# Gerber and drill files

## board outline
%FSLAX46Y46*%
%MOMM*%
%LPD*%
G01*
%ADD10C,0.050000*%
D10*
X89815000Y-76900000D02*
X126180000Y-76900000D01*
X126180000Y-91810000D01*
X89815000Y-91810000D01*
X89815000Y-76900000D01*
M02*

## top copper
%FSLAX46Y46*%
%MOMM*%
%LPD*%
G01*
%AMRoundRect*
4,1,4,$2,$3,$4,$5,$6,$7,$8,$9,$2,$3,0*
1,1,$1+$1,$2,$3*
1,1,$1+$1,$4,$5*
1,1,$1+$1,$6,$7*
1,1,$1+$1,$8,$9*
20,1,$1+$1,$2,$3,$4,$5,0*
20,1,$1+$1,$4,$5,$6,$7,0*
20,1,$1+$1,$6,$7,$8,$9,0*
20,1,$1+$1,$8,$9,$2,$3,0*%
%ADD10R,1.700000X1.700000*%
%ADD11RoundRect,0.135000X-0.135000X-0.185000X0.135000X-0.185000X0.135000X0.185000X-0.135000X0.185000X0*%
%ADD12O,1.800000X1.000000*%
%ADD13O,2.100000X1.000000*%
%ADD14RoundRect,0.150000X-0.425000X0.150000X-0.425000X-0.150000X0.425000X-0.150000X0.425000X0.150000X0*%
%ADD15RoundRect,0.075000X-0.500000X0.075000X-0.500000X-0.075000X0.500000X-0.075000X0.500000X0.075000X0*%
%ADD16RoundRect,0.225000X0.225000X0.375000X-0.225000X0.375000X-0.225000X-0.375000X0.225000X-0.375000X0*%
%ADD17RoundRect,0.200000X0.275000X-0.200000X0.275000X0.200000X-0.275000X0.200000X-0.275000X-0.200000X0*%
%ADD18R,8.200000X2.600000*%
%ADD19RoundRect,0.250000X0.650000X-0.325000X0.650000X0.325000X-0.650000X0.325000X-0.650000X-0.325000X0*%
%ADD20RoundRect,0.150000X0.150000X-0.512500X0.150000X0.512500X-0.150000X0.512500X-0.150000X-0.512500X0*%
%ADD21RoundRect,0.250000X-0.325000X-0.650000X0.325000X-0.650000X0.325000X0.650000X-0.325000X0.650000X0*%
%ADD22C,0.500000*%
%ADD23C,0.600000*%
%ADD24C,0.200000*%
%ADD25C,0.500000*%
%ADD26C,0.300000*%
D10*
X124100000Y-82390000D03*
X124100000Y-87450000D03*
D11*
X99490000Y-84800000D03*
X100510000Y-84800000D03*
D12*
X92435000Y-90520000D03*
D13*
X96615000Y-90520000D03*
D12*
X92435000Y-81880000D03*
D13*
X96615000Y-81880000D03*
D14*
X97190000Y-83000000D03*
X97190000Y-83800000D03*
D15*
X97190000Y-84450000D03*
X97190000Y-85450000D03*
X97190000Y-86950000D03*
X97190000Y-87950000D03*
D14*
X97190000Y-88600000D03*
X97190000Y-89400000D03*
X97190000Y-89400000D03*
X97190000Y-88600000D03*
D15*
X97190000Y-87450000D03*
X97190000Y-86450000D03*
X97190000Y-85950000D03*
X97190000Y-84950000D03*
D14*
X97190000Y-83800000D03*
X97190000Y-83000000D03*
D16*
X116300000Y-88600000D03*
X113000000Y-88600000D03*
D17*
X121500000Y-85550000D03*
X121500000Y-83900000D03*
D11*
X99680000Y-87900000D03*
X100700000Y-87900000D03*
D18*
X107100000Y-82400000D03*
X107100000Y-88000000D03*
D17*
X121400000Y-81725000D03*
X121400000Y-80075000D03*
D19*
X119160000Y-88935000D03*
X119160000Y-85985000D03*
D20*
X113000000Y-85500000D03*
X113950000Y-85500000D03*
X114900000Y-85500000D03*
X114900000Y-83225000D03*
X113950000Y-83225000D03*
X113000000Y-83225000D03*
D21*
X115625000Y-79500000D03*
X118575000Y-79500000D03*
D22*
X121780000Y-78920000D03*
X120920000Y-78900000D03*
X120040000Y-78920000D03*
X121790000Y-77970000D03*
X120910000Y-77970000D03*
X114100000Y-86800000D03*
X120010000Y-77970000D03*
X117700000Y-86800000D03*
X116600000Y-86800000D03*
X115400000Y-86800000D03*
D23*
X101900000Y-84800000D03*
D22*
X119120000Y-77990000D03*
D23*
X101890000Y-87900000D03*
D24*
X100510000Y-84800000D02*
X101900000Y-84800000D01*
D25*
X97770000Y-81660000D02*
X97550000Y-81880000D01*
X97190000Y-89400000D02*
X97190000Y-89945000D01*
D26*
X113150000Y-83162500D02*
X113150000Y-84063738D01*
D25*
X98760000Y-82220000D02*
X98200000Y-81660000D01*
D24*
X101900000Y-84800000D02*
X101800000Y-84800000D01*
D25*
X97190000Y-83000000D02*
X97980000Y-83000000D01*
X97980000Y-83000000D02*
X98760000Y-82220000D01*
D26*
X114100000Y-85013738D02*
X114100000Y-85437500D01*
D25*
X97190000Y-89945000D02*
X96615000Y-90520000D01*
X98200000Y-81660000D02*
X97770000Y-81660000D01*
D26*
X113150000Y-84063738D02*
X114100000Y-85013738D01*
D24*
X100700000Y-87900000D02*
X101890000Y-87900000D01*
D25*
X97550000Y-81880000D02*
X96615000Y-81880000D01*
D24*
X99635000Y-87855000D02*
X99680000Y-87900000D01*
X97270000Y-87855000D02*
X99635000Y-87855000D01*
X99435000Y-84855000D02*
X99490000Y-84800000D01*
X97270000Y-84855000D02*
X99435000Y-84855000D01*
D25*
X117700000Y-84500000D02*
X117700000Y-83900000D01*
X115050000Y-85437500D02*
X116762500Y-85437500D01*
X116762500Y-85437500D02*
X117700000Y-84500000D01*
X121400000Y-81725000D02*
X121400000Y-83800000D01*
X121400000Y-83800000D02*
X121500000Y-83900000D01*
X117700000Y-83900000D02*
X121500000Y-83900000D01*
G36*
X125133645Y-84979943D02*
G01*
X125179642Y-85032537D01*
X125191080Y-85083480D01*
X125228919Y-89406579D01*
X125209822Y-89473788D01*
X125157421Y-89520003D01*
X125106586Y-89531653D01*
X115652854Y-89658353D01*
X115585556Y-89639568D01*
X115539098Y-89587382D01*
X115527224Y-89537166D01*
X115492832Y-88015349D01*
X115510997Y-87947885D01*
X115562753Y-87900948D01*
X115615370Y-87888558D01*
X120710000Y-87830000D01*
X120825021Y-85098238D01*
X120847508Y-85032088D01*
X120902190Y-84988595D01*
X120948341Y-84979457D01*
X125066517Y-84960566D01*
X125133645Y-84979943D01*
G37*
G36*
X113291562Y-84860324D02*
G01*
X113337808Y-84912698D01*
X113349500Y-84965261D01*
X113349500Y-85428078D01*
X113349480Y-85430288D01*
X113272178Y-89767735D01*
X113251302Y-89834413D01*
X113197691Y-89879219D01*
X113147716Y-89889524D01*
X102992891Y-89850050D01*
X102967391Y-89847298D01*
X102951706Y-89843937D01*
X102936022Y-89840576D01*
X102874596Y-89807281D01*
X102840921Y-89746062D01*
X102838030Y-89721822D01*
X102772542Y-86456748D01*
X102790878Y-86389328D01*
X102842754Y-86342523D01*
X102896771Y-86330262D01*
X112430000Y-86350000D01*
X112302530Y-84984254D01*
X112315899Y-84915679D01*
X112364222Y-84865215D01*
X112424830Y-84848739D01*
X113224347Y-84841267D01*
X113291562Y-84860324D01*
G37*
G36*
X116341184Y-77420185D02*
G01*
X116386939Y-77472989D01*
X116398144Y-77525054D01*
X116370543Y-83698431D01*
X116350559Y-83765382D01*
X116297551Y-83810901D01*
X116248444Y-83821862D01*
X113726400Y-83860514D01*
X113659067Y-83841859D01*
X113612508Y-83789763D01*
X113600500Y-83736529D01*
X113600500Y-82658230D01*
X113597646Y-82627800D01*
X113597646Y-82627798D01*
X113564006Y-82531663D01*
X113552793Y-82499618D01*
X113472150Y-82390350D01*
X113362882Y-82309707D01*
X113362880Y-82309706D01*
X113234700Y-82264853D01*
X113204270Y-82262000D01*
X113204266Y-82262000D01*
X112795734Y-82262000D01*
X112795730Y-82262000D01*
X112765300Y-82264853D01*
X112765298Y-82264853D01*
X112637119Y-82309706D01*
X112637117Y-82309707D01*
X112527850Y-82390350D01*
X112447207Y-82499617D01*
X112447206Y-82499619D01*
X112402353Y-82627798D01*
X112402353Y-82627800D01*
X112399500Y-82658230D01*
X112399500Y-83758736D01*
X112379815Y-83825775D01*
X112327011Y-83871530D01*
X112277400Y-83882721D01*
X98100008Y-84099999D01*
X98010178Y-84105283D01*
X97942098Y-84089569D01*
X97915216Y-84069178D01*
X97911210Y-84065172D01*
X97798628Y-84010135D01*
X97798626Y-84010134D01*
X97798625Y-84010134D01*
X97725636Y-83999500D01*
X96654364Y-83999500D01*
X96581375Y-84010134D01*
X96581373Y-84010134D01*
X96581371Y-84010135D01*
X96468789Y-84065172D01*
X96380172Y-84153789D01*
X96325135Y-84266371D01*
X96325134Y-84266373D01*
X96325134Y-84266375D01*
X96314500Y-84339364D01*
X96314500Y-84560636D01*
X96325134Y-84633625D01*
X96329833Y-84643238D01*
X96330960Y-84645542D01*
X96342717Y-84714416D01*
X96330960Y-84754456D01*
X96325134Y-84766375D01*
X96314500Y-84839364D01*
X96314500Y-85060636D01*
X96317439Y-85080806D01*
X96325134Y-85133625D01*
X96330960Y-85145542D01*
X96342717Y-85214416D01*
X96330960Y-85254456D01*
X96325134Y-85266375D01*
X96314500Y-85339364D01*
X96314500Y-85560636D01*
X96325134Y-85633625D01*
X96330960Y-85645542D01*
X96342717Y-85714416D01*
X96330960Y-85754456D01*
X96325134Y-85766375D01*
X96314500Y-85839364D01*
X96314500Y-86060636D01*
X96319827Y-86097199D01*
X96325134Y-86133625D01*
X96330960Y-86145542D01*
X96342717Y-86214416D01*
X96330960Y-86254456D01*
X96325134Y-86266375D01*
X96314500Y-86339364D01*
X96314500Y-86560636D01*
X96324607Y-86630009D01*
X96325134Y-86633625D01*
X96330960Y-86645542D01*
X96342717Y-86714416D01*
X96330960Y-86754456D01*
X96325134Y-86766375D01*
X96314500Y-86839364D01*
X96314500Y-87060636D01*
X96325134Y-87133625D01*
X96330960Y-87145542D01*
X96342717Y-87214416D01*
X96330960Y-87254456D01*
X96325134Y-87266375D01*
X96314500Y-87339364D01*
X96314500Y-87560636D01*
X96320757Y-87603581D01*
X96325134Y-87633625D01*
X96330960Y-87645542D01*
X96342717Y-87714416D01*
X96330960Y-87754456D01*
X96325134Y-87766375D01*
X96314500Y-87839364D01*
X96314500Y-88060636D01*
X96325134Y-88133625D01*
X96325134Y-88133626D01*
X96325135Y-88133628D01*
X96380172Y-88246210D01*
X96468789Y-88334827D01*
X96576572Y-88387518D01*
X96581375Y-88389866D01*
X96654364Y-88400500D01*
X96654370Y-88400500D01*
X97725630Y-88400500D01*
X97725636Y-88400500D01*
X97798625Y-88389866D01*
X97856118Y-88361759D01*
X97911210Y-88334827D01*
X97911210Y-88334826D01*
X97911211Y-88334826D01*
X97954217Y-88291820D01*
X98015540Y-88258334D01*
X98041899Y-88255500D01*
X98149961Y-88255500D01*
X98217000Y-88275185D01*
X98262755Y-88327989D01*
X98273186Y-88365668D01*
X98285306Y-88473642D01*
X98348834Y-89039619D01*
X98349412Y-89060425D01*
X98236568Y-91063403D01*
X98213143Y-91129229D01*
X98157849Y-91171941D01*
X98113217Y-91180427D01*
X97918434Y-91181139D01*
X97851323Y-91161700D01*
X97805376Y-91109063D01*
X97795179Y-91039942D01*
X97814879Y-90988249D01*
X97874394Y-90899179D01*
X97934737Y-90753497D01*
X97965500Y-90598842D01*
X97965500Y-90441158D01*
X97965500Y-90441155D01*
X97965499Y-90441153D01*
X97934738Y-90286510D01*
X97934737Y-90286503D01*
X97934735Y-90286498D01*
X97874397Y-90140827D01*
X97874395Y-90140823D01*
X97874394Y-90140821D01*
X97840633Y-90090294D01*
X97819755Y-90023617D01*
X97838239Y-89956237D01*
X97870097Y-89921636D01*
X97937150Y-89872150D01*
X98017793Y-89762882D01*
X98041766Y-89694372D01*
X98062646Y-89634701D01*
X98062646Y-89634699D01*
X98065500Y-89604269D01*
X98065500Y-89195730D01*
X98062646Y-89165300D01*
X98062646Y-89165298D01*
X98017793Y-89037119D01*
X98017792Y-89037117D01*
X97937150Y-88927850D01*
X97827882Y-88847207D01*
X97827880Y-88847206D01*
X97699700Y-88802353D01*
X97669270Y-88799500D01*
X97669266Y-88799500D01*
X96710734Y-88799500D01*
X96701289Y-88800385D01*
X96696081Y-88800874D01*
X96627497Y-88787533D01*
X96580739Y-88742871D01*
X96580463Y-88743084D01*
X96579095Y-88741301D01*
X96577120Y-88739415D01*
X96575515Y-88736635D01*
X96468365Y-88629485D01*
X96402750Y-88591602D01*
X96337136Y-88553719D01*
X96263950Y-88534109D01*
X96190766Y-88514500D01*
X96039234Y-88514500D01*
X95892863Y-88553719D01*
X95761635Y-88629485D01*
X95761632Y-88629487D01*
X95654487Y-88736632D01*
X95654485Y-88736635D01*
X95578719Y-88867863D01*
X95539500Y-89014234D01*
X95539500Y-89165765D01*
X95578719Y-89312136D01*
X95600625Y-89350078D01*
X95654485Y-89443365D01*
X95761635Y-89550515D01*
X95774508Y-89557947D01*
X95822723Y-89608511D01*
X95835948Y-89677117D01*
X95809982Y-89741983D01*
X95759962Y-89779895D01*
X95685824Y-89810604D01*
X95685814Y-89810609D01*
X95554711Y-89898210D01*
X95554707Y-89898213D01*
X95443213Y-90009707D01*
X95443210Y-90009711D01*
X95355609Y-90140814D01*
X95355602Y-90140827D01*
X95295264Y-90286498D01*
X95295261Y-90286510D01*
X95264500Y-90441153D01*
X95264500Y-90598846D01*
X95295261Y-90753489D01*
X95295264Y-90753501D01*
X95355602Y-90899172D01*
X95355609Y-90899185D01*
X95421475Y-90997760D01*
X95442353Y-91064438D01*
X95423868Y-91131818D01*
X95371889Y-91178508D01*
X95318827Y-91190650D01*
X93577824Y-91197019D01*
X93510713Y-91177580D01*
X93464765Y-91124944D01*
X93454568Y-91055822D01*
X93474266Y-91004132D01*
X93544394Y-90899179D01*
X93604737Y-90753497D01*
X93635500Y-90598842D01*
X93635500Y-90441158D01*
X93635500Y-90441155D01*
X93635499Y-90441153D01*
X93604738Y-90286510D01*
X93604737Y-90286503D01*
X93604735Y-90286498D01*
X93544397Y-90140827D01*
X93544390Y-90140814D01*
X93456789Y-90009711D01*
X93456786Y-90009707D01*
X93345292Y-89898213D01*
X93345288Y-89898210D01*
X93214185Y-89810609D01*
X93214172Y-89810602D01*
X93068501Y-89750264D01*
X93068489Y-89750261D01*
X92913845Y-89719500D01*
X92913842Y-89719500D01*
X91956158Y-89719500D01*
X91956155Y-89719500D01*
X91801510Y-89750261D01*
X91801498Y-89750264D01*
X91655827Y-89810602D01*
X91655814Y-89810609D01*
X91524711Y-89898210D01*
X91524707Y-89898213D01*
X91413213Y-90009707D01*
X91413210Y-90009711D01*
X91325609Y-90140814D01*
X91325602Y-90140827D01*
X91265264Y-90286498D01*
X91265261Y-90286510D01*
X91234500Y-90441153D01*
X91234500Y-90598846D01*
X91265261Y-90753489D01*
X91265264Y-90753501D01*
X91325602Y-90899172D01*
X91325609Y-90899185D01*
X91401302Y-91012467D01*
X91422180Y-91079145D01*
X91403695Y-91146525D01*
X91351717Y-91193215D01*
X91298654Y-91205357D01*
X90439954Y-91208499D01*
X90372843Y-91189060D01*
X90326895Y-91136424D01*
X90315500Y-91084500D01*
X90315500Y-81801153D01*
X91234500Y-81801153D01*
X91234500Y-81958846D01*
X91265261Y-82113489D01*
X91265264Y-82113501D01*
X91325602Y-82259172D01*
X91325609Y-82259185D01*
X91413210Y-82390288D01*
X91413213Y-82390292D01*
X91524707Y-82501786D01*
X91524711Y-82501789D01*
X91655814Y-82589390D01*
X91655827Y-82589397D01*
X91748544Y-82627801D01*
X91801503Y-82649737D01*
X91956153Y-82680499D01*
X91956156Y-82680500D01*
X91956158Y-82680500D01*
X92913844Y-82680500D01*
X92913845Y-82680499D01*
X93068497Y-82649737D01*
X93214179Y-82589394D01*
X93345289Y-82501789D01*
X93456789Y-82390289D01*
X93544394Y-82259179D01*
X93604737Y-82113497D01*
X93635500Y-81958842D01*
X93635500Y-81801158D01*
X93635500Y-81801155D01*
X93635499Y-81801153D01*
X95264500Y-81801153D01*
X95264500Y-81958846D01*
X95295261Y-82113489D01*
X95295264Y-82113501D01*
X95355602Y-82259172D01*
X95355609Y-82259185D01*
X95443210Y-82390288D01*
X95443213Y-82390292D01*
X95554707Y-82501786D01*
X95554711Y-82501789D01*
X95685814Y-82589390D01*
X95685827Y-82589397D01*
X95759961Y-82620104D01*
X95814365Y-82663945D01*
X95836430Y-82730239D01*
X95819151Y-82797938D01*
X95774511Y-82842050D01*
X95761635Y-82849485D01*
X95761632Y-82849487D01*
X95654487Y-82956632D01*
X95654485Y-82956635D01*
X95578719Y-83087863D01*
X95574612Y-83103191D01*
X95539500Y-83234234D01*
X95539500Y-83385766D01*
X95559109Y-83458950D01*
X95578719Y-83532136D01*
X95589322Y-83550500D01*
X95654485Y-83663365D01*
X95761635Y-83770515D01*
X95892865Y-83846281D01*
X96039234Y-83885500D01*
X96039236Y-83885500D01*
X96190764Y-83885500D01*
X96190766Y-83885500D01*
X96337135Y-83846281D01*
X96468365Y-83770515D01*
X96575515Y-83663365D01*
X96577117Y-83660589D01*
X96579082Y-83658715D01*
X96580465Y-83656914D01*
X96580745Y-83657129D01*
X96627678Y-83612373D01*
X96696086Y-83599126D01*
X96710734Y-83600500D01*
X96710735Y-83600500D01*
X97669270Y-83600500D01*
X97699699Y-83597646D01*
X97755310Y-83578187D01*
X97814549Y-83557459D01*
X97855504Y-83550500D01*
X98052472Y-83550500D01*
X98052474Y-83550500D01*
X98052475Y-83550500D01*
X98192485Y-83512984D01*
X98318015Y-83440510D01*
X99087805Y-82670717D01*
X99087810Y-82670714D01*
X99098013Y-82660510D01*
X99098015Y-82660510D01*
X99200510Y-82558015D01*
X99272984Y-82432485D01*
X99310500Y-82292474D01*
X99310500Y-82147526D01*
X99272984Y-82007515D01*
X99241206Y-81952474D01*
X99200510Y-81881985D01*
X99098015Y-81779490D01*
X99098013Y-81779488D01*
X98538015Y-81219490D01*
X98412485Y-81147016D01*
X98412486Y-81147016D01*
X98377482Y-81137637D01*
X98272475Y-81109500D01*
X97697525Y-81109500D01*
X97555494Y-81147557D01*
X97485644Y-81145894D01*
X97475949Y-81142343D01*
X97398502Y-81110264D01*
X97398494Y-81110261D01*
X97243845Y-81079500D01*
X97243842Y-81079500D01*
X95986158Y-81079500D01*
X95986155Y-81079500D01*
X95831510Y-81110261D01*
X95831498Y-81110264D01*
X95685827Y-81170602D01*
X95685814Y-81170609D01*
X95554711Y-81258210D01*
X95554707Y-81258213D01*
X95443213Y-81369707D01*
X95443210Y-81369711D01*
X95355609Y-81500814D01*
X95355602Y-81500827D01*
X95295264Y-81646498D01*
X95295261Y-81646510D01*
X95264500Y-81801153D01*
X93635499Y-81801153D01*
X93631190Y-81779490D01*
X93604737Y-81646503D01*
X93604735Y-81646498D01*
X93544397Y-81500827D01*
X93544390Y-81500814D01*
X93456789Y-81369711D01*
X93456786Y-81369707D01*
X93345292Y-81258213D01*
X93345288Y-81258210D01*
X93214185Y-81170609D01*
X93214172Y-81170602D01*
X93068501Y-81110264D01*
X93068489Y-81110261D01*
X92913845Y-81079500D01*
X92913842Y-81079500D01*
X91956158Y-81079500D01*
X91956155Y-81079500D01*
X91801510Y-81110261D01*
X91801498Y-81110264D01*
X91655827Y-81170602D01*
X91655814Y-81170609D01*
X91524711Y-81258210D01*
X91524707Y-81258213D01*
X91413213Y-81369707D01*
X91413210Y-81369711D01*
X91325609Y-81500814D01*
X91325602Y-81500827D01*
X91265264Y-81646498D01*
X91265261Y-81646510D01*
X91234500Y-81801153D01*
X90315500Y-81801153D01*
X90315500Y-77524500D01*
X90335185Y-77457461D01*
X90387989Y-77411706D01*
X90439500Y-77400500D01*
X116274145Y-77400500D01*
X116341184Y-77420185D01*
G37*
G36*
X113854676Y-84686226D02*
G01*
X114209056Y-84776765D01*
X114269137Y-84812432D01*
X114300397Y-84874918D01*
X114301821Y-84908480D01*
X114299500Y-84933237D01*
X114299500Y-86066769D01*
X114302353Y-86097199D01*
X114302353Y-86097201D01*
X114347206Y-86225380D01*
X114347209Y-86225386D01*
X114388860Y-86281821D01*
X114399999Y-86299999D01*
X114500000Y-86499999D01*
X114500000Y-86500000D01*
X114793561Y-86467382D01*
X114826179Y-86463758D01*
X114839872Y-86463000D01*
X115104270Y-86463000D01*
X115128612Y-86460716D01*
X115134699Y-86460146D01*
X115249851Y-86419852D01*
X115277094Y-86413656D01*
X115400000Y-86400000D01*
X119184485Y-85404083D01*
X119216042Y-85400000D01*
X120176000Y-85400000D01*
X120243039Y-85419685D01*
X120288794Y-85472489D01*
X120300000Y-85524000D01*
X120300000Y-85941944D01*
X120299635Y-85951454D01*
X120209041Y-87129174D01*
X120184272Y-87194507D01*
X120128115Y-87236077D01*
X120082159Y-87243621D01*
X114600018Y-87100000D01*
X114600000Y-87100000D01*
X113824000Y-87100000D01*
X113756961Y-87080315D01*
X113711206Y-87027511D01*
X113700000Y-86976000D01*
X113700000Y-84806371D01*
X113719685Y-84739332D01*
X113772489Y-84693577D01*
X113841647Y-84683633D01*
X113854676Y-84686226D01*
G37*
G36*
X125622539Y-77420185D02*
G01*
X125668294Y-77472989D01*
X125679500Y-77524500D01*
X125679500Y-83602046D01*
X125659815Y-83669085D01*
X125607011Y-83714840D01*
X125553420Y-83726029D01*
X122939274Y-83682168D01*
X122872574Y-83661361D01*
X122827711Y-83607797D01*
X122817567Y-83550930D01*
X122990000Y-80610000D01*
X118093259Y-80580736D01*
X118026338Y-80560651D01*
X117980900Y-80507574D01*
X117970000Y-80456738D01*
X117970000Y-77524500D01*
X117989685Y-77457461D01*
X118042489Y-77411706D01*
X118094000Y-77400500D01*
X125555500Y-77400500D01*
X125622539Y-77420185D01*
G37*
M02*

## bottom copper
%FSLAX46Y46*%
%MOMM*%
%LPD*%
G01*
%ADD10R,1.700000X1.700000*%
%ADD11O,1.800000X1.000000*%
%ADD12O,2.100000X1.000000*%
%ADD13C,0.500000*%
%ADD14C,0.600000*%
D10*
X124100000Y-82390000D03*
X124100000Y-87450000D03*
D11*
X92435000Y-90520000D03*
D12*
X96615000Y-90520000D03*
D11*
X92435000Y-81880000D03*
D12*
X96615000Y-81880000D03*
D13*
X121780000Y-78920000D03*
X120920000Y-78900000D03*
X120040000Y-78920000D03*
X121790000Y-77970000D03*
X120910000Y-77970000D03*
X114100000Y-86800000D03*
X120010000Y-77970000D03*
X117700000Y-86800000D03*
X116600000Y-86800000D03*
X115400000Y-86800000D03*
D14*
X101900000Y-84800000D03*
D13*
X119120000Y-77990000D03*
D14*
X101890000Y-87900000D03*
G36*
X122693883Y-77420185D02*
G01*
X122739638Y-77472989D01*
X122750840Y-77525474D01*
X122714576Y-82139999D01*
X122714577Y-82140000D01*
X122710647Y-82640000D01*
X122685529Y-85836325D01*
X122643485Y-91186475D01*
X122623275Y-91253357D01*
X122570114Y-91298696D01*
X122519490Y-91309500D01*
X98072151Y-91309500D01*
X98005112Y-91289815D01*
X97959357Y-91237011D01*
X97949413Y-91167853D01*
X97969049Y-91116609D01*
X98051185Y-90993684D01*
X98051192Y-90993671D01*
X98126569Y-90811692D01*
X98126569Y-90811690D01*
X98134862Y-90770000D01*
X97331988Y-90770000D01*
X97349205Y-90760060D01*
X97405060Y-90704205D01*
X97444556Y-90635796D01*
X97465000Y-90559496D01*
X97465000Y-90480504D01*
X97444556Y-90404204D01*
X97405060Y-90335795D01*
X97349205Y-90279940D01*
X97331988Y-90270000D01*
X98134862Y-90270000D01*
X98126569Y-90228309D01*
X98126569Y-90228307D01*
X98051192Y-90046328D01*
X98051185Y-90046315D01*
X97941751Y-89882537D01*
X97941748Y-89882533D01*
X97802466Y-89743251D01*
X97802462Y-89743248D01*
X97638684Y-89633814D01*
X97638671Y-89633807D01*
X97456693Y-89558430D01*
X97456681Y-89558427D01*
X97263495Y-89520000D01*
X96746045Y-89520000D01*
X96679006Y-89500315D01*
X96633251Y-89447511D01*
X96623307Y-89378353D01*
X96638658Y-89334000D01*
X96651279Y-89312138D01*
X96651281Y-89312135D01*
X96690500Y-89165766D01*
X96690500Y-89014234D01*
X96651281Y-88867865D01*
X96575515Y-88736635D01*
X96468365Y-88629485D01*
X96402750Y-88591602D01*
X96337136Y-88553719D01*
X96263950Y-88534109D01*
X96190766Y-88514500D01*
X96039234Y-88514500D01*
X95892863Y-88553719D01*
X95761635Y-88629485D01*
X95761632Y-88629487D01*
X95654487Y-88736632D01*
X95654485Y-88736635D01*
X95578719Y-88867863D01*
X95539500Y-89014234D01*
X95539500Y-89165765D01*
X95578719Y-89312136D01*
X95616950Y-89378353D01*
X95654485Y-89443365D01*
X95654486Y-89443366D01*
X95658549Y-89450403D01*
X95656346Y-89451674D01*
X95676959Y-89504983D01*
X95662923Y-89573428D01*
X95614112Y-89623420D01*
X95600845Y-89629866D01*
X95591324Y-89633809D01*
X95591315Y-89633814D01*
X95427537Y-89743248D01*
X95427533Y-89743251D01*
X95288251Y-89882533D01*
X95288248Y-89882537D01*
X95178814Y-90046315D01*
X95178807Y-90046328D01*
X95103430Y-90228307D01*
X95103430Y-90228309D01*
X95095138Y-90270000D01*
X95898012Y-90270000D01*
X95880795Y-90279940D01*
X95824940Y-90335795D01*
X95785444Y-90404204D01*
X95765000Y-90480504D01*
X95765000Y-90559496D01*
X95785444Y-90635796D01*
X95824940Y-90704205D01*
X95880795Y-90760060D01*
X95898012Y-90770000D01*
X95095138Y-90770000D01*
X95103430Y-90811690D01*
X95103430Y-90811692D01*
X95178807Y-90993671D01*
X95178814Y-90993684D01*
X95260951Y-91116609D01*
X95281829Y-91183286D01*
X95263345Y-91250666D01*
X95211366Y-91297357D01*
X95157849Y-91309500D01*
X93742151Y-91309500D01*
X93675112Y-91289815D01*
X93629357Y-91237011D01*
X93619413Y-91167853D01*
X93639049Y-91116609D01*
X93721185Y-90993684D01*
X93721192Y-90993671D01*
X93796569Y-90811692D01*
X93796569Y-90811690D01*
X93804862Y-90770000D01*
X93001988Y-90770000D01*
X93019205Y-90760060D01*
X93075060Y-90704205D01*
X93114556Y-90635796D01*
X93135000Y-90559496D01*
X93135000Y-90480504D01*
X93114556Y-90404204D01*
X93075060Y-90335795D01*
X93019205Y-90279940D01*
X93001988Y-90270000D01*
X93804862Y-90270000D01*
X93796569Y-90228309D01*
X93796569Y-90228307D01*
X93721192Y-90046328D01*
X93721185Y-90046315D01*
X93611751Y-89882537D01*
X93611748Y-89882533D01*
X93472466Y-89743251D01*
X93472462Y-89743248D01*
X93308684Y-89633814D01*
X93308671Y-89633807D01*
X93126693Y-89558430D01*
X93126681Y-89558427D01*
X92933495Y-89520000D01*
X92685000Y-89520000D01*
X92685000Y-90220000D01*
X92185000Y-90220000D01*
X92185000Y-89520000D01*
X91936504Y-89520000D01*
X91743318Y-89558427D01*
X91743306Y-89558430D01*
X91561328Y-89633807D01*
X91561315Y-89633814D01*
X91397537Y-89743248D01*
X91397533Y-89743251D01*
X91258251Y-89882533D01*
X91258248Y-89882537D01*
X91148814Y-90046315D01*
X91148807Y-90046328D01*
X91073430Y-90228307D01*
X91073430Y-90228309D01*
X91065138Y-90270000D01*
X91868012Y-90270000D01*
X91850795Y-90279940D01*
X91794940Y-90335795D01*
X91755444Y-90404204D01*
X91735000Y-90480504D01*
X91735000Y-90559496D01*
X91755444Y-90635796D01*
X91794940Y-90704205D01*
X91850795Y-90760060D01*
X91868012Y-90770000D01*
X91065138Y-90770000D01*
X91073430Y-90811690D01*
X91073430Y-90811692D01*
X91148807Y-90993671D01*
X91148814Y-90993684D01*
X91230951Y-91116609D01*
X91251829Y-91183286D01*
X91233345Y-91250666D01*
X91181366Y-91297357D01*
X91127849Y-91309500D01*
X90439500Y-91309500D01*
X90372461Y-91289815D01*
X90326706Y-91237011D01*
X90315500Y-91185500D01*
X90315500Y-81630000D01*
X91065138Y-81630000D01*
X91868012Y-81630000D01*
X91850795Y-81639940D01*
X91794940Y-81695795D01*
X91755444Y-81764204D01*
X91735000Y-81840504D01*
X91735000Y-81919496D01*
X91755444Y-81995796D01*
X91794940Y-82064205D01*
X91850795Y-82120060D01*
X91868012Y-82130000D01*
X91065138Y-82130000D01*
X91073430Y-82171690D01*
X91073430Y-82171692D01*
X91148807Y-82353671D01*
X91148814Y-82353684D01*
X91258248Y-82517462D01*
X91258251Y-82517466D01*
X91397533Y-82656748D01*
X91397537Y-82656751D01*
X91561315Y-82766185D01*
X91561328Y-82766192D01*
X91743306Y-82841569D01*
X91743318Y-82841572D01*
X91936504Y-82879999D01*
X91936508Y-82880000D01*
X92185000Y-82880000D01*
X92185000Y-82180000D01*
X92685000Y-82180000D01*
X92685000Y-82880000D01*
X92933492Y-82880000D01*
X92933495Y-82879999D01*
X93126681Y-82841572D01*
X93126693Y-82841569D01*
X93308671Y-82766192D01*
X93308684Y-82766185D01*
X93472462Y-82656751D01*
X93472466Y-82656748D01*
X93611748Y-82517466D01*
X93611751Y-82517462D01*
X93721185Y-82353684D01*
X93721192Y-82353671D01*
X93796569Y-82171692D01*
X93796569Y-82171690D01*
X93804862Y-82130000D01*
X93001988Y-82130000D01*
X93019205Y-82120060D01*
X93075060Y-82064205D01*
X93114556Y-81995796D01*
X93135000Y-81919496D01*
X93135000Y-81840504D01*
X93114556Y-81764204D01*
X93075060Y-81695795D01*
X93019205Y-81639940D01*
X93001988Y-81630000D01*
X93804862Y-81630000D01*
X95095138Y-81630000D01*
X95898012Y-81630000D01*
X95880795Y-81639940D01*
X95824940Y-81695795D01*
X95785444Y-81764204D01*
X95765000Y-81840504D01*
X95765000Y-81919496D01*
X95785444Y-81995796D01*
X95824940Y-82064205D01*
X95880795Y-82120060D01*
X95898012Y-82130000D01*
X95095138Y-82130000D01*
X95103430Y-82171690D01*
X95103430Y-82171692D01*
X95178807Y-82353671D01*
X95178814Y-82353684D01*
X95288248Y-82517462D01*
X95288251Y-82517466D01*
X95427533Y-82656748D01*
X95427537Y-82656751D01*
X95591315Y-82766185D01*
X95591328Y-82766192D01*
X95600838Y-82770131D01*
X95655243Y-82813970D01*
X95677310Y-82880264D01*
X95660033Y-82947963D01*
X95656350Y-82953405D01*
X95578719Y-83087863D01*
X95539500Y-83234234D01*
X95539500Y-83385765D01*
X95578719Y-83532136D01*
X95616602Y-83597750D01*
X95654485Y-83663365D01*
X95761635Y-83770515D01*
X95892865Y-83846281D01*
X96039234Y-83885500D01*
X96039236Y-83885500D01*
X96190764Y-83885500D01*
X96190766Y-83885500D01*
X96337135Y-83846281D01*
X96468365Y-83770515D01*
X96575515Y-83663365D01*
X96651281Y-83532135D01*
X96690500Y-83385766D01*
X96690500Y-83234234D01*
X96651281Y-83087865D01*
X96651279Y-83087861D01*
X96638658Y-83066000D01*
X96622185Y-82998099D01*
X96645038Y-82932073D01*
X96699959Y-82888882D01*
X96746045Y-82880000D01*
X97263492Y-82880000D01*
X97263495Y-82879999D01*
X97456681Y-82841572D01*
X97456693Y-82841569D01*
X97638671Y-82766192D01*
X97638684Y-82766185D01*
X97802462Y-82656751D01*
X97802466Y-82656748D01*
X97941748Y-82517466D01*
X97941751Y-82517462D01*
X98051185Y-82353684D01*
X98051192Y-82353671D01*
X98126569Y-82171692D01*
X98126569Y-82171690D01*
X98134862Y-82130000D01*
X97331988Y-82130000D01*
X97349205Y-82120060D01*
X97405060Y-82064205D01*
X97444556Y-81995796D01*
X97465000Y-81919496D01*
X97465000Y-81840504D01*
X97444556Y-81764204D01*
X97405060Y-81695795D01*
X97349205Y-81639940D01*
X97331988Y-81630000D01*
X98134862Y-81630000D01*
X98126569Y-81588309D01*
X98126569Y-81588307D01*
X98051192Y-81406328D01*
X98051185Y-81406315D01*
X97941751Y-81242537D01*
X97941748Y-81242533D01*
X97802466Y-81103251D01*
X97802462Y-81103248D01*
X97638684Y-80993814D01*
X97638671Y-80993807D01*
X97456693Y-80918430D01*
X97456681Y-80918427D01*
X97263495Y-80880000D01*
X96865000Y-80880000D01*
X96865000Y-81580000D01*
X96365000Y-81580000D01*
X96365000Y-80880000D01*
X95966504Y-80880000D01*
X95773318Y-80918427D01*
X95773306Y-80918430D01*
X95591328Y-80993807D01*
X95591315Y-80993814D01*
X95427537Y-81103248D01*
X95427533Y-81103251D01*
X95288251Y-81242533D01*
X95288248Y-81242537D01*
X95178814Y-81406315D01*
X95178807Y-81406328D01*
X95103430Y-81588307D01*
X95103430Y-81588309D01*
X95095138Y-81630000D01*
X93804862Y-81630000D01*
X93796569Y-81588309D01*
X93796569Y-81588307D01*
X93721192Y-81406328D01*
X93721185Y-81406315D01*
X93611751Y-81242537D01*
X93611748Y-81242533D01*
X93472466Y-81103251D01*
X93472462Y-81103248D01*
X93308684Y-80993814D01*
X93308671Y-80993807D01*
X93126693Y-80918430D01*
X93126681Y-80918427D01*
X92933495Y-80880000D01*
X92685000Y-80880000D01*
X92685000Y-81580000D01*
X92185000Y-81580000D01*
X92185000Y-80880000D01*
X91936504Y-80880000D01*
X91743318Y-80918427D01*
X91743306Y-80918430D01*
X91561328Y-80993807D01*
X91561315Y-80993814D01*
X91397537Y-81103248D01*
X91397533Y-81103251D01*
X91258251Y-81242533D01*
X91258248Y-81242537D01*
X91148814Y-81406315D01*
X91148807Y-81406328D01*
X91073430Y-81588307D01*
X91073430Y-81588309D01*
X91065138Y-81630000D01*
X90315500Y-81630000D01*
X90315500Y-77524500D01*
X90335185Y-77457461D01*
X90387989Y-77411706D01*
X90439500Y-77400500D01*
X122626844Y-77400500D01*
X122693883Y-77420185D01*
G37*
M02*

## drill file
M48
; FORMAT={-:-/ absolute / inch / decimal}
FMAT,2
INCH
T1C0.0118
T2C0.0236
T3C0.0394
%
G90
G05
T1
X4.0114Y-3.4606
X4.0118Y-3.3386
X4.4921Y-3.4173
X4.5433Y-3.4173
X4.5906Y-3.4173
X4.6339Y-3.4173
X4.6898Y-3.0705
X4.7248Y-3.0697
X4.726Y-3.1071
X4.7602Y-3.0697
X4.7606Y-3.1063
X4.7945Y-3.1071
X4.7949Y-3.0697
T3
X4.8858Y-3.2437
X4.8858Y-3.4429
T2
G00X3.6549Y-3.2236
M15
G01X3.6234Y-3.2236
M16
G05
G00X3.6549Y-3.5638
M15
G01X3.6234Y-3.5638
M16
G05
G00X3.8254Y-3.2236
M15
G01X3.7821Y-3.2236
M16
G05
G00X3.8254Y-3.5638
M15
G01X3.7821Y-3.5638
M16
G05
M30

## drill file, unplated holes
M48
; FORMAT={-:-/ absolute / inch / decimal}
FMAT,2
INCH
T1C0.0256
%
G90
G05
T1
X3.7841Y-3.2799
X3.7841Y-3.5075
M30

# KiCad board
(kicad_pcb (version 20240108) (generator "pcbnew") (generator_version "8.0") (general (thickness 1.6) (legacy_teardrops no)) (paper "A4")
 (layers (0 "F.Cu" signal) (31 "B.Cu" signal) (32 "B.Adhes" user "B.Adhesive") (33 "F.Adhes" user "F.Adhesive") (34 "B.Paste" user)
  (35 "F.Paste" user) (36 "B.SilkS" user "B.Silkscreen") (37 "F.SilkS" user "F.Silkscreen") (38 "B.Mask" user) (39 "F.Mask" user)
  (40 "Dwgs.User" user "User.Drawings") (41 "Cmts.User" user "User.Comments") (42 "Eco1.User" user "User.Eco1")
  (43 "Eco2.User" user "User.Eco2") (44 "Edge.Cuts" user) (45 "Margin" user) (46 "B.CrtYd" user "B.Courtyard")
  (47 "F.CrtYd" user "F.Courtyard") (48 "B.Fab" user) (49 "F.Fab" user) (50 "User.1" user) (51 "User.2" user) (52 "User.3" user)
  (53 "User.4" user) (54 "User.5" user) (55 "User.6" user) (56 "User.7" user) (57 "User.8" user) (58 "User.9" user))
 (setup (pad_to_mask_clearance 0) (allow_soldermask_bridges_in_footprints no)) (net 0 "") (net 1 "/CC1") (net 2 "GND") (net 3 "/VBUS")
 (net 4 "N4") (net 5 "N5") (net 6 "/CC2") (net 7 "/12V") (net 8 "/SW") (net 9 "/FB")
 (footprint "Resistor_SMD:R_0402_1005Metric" (layer "F.Cu") (at 100 84.8)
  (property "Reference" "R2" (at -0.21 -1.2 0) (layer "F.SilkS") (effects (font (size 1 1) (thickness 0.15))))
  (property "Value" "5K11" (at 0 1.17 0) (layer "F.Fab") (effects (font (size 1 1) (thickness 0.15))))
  (pad "1" smd roundrect (at -0.51 0) (size 0.54 0.64) (layers "F.Cu" "F.Paste" "F.Mask") (roundrect_rratio 0.25) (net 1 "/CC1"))
  (pad "2" smd roundrect (at 0.51 0) (size 0.54 0.64) (layers "F.Cu" "F.Paste" "F.Mask") (roundrect_rratio 0.25) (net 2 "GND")))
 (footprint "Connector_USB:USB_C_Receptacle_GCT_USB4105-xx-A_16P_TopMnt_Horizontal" (layer "F.Cu") (at 93.51 86.2 -90)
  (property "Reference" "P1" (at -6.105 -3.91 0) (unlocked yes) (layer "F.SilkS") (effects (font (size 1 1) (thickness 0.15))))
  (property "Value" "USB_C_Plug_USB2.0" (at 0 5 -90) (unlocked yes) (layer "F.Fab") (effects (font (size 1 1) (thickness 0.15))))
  (pad "" np_thru_hole circle (at -2.89 -2.605 270) (size 0.65 0.65) (drill 0.65) (layers "F&B.Cu" "*.Mask"))
  (pad "" np_thru_hole circle (at 2.89 -2.605 270) (size 0.65 0.65) (drill 0.65) (layers "F&B.Cu" "*.Mask"))
  (pad "A1" smd roundrect (at -3.2 -3.68 270) (size 0.6 1.15) (layers "F.Cu" "F.Paste" "F.Mask") (roundrect_rratio 0.25) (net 2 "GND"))
  (pad "A4" smd roundrect (at -2.4 -3.68 270) (size 0.6 1.15) (layers "F.Cu" "F.Paste" "F.Mask") (roundrect_rratio 0.25) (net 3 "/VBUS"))
  (pad "A5" smd roundrect (at -1.25 -3.68 270) (size 0.3 1.15) (layers "F.Cu" "F.Paste" "F.Mask") (roundrect_rratio 0.25) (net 1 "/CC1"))
  (pad "A6" smd roundrect (at -0.25 -3.68 270) (size 0.3 1.15) (layers "F.Cu" "F.Paste" "F.Mask") (roundrect_rratio 0.25) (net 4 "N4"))
  (pad "A7" smd roundrect (at 0.25 -3.68 270) (size 0.3 1.15) (layers "F.Cu" "F.Paste" "F.Mask") (roundrect_rratio 0.25) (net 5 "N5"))
  (pad "A8" smd roundrect (at 1.25 -3.68 270) (size 0.3 1.15) (layers "F.Cu" "F.Paste" "F.Mask") (roundrect_rratio 0.25))
  (pad "A9" smd roundrect (at 2.4 -3.68 270) (size 0.6 1.15) (layers "F.Cu" "F.Paste" "F.Mask") (roundrect_rratio 0.25) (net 3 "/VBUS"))
  (pad "A12" smd roundrect (at 3.2 -3.68 270) (size 0.6 1.15) (layers "F.Cu" "F.Paste" "F.Mask") (roundrect_rratio 0.25) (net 2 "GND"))
  (pad "B1" smd roundrect (at 3.2 -3.68 270) (size 0.6 1.15) (layers "F.Cu" "F.Paste" "F.Mask") (roundrect_rratio 0.25) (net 2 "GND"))
  (pad "B4" smd roundrect (at 2.4 -3.68 270) (size 0.6 1.15) (layers "F.Cu" "F.Paste" "F.Mask") (roundrect_rratio 0.25) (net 3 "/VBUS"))
  (pad "B5" smd roundrect (at 1.75 -3.68 270) (size 0.3 1.15) (layers "F.Cu" "F.Paste" "F.Mask") (roundrect_rratio 0.25) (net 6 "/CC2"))
  (pad "B6" smd roundrect (at 0.75 -3.68 270) (size 0.3 1.15) (layers "F.Cu" "F.Paste" "F.Mask") (roundrect_rratio 0.25))
  (pad "B7" smd roundrect (at -0.75 -3.68 270) (size 0.3 1.15) (layers "F.Cu" "F.Paste" "F.Mask") (roundrect_rratio 0.25))
  (pad "B8" smd roundrect (at -1.75 -3.68 270) (size 0.3 1.15) (layers "F.Cu" "F.Paste" "F.Mask") (roundrect_rratio 0.25))
  (pad "B9" smd roundrect (at -2.4 -3.68 270) (size 0.6 1.15) (layers "F.Cu" "F.Paste" "F.Mask") (roundrect_rratio 0.25) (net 3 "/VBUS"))
  (pad "B12" smd roundrect (at -3.2 -3.68 270) (size 0.6 1.15) (layers "F.Cu" "F.Paste" "F.Mask") (roundrect_rratio 0.25) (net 2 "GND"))
  (pad "S1" thru_hole oval (at -4.32 -3.105 270) (size 1 2.1) (drill oval 0.6 1.7) (layers "*.Cu" "*.Mask" "F.Paste")
   (remove_unused_layers no) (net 2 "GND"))
  (pad "S1" thru_hole oval (at -4.32 1.075 270) (size 1 1.8) (drill oval 0.6 1.4) (layers "*.Cu" "*.Mask" "F.Paste")
   (remove_unused_layers no) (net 2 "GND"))
  (pad "S1" thru_hole oval (at 4.32 -3.105 270) (size 1 2.1) (drill oval 0.6 1.7) (layers "*.Cu" "*.Mask" "F.Paste")
   (remove_unused_layers no) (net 2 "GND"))
  (pad "S1" thru_hole oval (at 4.32 1.075 270) (size 1 1.8) (drill oval 0.6 1.4) (layers "*.Cu" "*.Mask" "F.Paste")
   (remove_unused_layers no) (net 2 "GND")))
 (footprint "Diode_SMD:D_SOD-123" (layer "F.Cu") (at 114.65 88.6 180)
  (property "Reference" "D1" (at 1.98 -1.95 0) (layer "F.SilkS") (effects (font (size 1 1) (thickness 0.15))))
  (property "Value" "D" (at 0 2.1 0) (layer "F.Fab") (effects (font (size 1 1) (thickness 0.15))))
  (pad "1" smd roundrect (at -1.65 0 180) (size 0.9 1.2) (layers "F.Cu" "F.Paste" "F.Mask") (roundrect_rratio 0.25) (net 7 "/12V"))
  (pad "2" smd roundrect (at 1.65 0 180) (size 0.9 1.2) (layers "F.Cu" "F.Paste" "F.Mask") (roundrect_rratio 0.25) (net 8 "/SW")))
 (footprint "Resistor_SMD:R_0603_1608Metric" (layer "F.Cu") (at 121.5 84.725 90)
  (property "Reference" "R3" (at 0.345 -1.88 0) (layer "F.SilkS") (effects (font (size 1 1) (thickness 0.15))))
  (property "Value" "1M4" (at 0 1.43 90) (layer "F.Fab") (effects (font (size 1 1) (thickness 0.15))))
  (pad "1" smd roundrect (at -0.825 0 90) (size 0.8 0.95) (layers "F.Cu" "F.Paste" "F.Mask") (roundrect_rratio 0.25) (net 7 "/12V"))
  (pad "2" smd roundrect (at 0.825 0 90) (size 0.8 0.95) (layers "F.Cu" "F.Paste" "F.Mask") (roundrect_rratio 0.25) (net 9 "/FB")))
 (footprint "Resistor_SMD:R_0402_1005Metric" (layer "F.Cu") (at 100.19 87.9)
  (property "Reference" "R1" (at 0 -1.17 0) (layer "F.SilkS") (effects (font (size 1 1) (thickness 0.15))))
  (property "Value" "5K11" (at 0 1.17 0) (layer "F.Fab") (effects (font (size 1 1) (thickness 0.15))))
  (pad "1" smd roundrect (at -0.51 0) (size 0.54 0.64) (layers "F.Cu" "F.Paste" "F.Mask") (roundrect_rratio 0.25) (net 6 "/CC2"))
  (pad "2" smd roundrect (at 0.51 0) (size 0.54 0.64) (layers "F.Cu" "F.Paste" "F.Mask") (roundrect_rratio 0.25) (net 2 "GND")))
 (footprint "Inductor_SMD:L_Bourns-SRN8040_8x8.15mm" (layer "F.Cu") (at 107.1 85.2 -90)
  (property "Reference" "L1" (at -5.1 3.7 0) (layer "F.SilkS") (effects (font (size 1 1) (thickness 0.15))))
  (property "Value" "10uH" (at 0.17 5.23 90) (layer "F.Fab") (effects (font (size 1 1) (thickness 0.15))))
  (pad "1" smd rect (at -2.8 0 270) (size 2.6 8.2) (layers "F.Cu" "F.Paste" "F.Mask") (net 3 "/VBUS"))
  (pad "2" smd rect (at 2.8 0 270) (size 2.6 8.2) (layers "F.Cu" "F.Paste" "F.Mask") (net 8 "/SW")))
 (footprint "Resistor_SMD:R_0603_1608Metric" (layer "F.Cu") (at 121.4 80.9 90)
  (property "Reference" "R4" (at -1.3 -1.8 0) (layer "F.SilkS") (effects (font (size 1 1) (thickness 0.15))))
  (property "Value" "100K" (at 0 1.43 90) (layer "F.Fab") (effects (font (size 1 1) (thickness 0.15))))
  (pad "1" smd roundrect (at -0.825 0 90) (size 0.8 0.95) (layers "F.Cu" "F.Paste" "F.Mask") (roundrect_rratio 0.25) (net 9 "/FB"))
  (pad "2" smd roundrect (at 0.825 0 90) (size 0.8 0.95) (layers "F.Cu" "F.Paste" "F.Mask") (roundrect_rratio 0.25) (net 2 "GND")))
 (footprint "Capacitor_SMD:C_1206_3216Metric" (layer "F.Cu") (at 119.16 87.46 90)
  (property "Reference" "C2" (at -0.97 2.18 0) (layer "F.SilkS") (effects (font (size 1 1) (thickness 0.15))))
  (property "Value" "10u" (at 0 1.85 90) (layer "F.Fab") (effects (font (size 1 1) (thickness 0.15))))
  (pad "1" smd roundrect (at -1.475 0 90) (size 1.15 1.8) (layers "F.Cu" "F.Paste" "F.Mask") (roundrect_rratio 0.217391) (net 7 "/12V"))
  (pad "2" smd roundrect (at 1.475 0 90) (size 1.15 1.8) (layers "F.Cu" "F.Paste" "F.Mask") (roundrect_rratio 0.217391) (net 2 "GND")))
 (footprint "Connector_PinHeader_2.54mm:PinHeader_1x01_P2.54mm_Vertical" (layer "F.Cu") (at 124.1 82.39)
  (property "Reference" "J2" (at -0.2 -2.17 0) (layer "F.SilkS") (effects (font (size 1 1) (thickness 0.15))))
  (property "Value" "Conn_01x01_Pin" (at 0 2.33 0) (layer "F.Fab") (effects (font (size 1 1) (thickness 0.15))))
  (pad "1" thru_hole rect (at 0 0) (size 1.7 1.7) (drill 1) (layers "*.Cu" "*.Mask") (remove_unused_layers no) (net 2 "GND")))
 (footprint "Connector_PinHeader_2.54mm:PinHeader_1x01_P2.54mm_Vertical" (layer "F.Cu") (at 124.1 87.45)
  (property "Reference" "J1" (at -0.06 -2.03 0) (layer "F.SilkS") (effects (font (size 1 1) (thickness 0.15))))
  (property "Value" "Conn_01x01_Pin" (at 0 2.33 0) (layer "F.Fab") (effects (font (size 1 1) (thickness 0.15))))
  (pad "1" thru_hole rect (at 0 0) (size 1.7 1.7) (drill 1) (layers "*.Cu" "*.Mask") (remove_unused_layers no) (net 7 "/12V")))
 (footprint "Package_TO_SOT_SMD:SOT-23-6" (layer "F.Cu") (at 113.95 84.3625 90)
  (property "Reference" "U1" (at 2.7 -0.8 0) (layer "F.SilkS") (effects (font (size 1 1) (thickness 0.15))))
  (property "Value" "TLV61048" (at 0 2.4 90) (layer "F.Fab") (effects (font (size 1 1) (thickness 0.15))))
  (pad "1" smd roundrect (at -1.1375 -0.95 90) (size 1.325 0.6) (layers "F.Cu" "F.Paste" "F.Mask") (roundrect_rratio 0.25) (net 8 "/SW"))
  (pad "2" smd roundrect (at -1.1375 0 90) (size 1.325 0.6) (layers "F.Cu" "F.Paste" "F.Mask") (roundrect_rratio 0.25) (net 2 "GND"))
  (pad "3" smd roundrect (at -1.1375 0.95 90) (size 1.325 0.6) (layers "F.Cu" "F.Paste" "F.Mask") (roundrect_rratio 0.25) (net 9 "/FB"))
  (pad "4" smd roundrect (at 1.1375 0.95 90) (size 1.325 0.6) (layers "F.Cu" "F.Paste" "F.Mask") (roundrect_rratio 0.25) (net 3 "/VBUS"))
  (pad "5" smd roundrect (at 1.1375 0 90) (size 1.325 0.6) (layers "F.Cu" "F.Paste" "F.Mask") (roundrect_rratio 0.25) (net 3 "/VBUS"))
  (pad "6" smd roundrect (at 1.1375 -0.95 90) (size 1.325 0.6) (layers "F.Cu" "F.Paste" "F.Mask") (roundrect_rratio 0.25) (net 2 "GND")))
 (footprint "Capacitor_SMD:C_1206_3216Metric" (layer "F.Cu") (at 117.1 79.5)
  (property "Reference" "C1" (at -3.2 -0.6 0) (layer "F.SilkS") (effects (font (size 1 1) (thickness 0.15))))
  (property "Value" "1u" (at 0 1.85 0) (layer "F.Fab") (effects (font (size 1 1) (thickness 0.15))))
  (pad "1" smd roundrect (at -1.475 0) (size 1.15 1.8) (layers "F.Cu" "F.Paste" "F.Mask") (roundrect_rratio 0.217391) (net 3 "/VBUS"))
  (pad "2" smd roundrect (at 1.475 0) (size 1.15 1.8) (layers "F.Cu" "F.Paste" "F.Mask") (roundrect_rratio 0.217391) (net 2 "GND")))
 (gr_rect (start 89.815 76.9) (end 126.18 91.81) (stroke (width 0.05) (type default)) (fill none) (layer "Edge.Cuts"))
 (segment (start 100.51 84.8) (end 101.9 84.8) (width 0.2) (layer "F.Cu") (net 2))
 (segment (start 97.77 81.66) (end 97.55 81.88) (width 0.5) (layer "F.Cu") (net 2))
 (segment (start 97.19 89.4) (end 97.19 89.945) (width 0.5) (layer "F.Cu") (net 2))
 (segment (start 113.15 83.1625) (end 113.15 84.063738) (width 0.3) (layer "F.Cu") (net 2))
 (segment (start 98.76 82.22) (end 98.2 81.66) (width 0.5) (layer "F.Cu") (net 2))
 (segment (start 101.9 84.8) (end 101.8 84.8) (width 0.2) (layer "F.Cu") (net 2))
 (segment (start 97.19 83) (end 97.98 83) (width 0.5) (layer "F.Cu") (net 2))
 (segment (start 97.98 83) (end 98.76 82.22) (width 0.5) (layer "F.Cu") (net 2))
 (segment (start 114.1 85.013738) (end 114.1 85.4375) (width 0.3) (layer "F.Cu") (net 2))
 (segment (start 97.19 89.945) (end 96.615 90.52) (width 0.5) (layer "F.Cu") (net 2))
 (segment (start 98.2 81.66) (end 97.77 81.66) (width 0.5) (layer "F.Cu") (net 2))
 (segment (start 113.15 84.063738) (end 114.1 85.013738) (width 0.3) (layer "F.Cu") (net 2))
 (segment (start 100.7 87.9) (end 101.89 87.9) (width 0.2) (layer "F.Cu") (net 2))
 (segment (start 97.55 81.88) (end 96.615 81.88) (width 0.5) (layer "F.Cu") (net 2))
 (via (at 120.04 78.92) (size 0.5) (drill 0.3) (layers "F.Cu" "B.Cu") (free yes) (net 2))
 (via (at 114.1 86.8) (size 0.5) (drill 0.3) (layers "F.Cu" "B.Cu") (free yes) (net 2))
 (via (at 120.01 77.97) (size 0.5) (drill 0.3) (layers "F.Cu" "B.Cu") (free yes) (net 2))
 (via (at 117.7 86.8) (size 0.5) (drill 0.3) (layers "F.Cu" "B.Cu") (free yes) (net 2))
 (via (at 121.79 77.97) (size 0.5) (drill 0.3) (layers "F.Cu" "B.Cu") (free yes) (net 2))
 (via (at 120.91 77.97) (size 0.5) (drill 0.3) (layers "F.Cu" "B.Cu") (free yes) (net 2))
 (via (at 116.6 86.8) (size 0.5) (drill 0.3) (layers "F.Cu" "B.Cu") (free yes) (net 2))
 (via (at 115.4 86.8) (size 0.5) (drill 0.3) (layers "F.Cu" "B.Cu") (free yes) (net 2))
 (via (at 101.9 84.8) (size 0.6) (drill 0.3) (layers "F.Cu" "B.Cu") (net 2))
 (via (at 119.12 77.99) (size 0.5) (drill 0.3) (layers "F.Cu" "B.Cu") (free yes) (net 2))
 (via (at 121.78 78.92) (size 0.5) (drill 0.3) (layers "F.Cu" "B.Cu") (free yes) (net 2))
 (via (at 101.89 87.9) (size 0.6) (drill 0.3) (layers "F.Cu" "B.Cu") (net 2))
 (via (at 120.92 78.9) (size 0.5) (drill 0.3) (layers "F.Cu" "B.Cu") (free yes) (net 2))
 (segment (start 99.635 87.855) (end 99.68 87.9) (width 0.2) (layer "F.Cu") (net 6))
 (segment (start 97.27 87.855) (end 99.635 87.855) (width 0.2) (layer "F.Cu") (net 6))
 (segment (start 99.435 84.855) (end 99.49 84.8) (width 0.2) (layer "F.Cu") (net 1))
 (segment (start 97.27 84.855) (end 99.435 84.855) (width 0.2) (layer "F.Cu") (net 1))
 (segment (start 117.7 84.5) (end 117.7 83.9) (width 0.5) (layer "F.Cu") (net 9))
 (segment (start 115.05 85.4375) (end 116.7625 85.4375) (width 0.5) (layer "F.Cu") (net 9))
 (segment (start 116.7625 85.4375) (end 117.7 84.5) (width 0.5) (layer "F.Cu") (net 9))
 (segment (start 121.4 81.725) (end 121.4 83.8) (width 0.5) (layer "F.Cu") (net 9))
 (segment (start 121.4 83.8) (end 121.5 83.9) (width 0.5) (layer "F.Cu") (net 9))
 (segment (start 117.7 83.9) (end 121.5 83.9) (width 0.5) (layer "F.Cu") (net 9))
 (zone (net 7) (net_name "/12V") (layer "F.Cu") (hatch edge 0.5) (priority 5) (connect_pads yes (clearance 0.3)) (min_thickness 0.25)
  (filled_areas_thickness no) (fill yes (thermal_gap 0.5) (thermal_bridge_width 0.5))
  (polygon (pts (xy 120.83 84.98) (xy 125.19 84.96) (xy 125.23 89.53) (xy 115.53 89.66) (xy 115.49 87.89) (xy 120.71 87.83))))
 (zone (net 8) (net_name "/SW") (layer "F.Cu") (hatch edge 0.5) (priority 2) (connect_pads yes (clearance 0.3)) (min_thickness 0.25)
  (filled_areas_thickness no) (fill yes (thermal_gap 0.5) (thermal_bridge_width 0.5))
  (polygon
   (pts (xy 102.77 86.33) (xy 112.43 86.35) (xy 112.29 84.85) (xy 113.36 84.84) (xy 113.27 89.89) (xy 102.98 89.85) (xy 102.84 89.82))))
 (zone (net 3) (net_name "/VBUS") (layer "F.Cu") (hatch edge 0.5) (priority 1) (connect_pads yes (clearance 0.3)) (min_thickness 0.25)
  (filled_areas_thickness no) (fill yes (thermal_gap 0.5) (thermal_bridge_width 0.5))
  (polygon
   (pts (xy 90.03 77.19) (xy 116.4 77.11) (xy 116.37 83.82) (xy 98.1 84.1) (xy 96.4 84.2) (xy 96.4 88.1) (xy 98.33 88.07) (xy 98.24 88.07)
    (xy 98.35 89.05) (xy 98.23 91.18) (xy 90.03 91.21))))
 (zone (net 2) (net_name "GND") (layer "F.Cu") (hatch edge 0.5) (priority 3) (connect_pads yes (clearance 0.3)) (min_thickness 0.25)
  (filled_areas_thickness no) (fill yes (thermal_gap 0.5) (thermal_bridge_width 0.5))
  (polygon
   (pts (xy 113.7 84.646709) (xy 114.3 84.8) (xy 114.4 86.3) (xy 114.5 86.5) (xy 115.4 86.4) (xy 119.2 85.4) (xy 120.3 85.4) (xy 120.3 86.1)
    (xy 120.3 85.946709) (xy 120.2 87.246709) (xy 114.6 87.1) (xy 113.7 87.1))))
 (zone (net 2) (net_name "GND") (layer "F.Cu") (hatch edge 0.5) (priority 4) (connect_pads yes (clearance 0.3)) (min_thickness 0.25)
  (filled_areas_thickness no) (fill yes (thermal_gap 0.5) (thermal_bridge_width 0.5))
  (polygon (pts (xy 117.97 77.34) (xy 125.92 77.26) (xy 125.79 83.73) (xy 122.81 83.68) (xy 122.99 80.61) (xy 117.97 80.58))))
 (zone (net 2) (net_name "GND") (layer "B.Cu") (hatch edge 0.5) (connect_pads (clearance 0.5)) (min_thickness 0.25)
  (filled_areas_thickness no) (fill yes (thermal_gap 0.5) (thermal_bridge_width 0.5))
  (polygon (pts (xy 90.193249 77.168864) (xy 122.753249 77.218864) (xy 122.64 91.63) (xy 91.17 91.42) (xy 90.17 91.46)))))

